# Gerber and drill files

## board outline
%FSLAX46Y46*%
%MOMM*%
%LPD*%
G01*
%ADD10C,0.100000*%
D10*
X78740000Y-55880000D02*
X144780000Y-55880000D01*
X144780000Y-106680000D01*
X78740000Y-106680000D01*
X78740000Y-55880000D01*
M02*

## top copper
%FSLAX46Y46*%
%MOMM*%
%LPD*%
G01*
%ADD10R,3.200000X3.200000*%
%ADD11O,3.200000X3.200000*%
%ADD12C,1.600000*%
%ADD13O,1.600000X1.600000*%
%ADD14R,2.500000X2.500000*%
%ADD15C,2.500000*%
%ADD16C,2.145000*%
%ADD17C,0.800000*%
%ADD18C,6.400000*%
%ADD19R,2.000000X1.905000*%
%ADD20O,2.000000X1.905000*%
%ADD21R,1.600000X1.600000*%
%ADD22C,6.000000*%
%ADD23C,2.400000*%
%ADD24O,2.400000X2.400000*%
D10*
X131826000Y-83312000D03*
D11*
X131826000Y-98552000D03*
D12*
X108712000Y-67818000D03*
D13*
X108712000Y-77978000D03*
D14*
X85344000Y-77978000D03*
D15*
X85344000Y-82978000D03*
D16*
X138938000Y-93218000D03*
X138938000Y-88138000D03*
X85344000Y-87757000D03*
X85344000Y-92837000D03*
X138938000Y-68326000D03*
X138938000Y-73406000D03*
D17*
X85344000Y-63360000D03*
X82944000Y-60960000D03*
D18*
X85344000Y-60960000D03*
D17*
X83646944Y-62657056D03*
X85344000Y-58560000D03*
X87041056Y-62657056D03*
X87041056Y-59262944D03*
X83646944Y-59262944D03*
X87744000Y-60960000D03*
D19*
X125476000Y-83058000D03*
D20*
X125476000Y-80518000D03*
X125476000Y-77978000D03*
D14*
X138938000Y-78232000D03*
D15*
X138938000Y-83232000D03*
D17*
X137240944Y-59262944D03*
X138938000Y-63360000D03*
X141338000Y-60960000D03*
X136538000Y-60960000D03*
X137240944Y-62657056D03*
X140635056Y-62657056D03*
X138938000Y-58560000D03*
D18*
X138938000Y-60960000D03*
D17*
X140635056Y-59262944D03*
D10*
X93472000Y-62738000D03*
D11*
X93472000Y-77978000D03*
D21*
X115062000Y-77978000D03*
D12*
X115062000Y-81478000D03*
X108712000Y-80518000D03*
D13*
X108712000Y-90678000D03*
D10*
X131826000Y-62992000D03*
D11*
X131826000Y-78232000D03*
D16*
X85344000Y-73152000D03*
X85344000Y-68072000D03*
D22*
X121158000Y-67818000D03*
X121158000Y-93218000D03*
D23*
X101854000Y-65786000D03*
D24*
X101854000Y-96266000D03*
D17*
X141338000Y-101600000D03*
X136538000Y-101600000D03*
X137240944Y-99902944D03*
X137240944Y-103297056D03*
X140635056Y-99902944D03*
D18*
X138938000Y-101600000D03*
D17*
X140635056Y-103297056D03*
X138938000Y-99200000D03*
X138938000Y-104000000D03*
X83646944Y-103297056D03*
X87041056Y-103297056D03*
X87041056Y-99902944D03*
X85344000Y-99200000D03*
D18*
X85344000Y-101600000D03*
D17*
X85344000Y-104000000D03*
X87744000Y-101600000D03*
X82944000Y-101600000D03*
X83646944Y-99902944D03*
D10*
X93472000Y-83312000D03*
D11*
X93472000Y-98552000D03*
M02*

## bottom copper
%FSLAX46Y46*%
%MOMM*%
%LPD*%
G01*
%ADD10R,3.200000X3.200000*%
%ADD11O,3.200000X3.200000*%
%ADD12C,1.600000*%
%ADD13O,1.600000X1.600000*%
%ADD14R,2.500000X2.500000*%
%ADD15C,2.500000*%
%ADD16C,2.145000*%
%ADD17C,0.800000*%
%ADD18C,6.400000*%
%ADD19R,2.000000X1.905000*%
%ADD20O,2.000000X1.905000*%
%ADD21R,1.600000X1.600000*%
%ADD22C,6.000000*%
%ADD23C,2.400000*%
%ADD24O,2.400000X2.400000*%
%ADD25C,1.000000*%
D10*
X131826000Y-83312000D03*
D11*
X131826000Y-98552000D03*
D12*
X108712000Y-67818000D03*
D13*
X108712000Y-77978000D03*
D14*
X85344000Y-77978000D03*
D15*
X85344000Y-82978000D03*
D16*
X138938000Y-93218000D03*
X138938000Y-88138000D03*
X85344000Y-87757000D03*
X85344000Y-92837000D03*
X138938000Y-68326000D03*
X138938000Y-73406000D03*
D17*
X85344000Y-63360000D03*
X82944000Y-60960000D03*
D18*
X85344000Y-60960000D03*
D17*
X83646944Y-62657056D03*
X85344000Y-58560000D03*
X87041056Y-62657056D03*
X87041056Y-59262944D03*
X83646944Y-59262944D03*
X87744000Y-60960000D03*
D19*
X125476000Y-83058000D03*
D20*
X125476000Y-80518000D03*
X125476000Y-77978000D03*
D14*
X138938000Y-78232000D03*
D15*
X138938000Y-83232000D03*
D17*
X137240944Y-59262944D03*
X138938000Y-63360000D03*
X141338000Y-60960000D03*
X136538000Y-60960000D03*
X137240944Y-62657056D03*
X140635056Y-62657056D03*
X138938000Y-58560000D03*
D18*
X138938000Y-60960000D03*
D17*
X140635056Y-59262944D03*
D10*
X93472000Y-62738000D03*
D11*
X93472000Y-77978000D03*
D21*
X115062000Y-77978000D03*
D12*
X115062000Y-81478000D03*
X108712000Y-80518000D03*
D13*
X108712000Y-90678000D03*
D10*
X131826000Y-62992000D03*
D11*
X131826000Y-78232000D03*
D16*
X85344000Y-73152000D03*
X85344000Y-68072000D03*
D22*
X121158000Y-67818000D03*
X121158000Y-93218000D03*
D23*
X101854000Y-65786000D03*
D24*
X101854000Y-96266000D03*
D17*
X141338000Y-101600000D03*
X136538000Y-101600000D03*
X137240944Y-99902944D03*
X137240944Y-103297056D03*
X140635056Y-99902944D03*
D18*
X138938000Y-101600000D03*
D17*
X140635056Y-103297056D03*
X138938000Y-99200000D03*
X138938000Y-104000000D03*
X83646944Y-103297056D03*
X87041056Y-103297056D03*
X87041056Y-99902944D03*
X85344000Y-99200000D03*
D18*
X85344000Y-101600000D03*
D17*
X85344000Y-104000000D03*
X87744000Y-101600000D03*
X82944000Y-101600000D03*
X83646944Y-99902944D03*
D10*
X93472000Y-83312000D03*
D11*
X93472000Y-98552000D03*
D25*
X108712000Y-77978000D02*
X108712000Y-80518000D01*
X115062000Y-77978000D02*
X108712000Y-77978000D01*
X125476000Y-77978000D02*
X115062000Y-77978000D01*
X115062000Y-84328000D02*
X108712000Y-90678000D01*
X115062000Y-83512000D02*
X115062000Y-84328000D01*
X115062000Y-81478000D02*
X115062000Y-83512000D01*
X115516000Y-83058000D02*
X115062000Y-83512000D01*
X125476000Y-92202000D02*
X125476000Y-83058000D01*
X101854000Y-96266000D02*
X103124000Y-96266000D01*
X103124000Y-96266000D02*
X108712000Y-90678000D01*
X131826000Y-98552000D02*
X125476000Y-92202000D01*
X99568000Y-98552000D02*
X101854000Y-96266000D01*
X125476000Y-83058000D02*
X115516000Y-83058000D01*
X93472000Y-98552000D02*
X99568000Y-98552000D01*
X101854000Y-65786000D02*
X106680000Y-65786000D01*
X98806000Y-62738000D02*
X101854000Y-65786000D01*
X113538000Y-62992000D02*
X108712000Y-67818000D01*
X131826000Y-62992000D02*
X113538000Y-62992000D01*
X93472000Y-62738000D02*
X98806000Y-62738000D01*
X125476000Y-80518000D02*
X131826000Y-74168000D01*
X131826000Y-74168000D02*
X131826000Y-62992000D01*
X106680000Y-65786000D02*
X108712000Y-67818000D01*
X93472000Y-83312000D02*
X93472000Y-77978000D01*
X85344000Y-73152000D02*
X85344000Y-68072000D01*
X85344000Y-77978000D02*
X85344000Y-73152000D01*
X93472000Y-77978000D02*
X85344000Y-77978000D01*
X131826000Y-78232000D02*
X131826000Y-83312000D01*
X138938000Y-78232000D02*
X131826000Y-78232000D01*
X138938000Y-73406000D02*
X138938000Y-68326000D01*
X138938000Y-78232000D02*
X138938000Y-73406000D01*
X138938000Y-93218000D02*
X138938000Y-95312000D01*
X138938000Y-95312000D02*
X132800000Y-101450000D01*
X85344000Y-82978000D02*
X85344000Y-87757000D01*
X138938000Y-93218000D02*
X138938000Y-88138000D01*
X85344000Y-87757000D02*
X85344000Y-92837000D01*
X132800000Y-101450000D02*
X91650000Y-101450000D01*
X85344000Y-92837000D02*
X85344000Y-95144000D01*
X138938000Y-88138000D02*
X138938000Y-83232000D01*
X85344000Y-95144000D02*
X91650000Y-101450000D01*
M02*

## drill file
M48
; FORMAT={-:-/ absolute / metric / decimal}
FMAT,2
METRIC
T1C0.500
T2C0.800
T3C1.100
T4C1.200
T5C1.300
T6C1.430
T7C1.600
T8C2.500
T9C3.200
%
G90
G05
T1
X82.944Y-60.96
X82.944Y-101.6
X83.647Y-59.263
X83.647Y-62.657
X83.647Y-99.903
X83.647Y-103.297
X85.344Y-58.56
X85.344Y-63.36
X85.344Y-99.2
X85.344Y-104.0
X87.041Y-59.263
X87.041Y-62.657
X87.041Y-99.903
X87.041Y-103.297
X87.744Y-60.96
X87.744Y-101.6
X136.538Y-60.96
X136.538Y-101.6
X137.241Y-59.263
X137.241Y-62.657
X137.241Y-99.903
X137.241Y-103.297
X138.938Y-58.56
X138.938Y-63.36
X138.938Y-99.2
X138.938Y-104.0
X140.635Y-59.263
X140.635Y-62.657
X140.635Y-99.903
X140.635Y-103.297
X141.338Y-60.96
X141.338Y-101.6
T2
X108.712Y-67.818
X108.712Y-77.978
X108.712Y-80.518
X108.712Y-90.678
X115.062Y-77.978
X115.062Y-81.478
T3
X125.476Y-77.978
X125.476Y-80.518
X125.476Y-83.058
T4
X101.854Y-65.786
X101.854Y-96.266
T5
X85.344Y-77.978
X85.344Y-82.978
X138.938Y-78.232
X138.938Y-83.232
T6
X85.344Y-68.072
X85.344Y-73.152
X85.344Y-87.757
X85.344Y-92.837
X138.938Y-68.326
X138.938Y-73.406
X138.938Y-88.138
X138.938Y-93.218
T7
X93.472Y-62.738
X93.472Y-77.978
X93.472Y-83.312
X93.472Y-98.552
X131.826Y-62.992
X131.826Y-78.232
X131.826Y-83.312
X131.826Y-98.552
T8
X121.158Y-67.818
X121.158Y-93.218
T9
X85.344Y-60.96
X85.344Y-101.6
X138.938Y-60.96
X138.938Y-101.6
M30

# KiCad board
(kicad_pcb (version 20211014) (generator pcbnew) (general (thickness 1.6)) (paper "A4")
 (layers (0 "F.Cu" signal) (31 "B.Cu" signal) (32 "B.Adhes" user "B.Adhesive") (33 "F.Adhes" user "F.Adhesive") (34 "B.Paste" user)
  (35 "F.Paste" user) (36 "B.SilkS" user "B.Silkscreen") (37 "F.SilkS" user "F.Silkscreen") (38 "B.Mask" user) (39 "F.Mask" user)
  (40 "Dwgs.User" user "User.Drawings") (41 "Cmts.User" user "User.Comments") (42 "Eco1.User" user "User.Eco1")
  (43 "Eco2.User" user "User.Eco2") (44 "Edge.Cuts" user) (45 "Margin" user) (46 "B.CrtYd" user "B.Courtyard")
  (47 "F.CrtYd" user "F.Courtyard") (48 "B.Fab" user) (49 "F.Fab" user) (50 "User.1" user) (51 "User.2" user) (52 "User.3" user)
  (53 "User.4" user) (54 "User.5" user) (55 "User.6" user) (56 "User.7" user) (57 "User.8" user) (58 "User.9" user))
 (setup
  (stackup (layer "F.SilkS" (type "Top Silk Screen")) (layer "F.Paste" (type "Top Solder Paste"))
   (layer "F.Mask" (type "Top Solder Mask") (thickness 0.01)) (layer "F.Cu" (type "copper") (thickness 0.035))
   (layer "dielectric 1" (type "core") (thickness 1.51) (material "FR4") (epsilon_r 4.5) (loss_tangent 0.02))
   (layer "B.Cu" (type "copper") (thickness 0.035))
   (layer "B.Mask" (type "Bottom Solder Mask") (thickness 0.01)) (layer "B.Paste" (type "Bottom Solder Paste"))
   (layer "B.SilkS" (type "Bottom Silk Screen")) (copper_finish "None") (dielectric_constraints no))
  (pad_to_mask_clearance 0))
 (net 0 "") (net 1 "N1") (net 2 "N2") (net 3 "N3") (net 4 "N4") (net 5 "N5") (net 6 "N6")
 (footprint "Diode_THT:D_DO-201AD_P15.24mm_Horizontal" (layer "F.Cu") (at 131.826 83.312 -90)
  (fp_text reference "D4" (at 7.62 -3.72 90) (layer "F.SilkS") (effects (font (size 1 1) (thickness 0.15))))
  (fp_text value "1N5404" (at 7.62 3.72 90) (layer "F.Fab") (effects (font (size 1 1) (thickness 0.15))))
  (pad "1" thru_hole rect (at 0 0 270) (size 3.2 3.2) (drill 1.6) (layers *.Cu *.Mask) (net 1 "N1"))
  (pad "2" thru_hole oval (at 15.24 0 270) (size 3.2 3.2) (drill 1.6) (layers *.Cu *.Mask) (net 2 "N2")))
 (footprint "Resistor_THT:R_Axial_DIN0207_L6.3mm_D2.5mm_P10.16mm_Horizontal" (layer "F.Cu") (at 108.712 67.818 -90)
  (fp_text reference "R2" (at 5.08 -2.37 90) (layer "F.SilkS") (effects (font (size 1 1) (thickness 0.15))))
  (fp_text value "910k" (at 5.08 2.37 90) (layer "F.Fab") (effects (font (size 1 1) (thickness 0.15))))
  (pad "1" thru_hole circle (at 0 0 270) (size 1.6 1.6) (drill 0.8) (layers *.Cu *.Mask) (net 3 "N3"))
  (pad "2" thru_hole oval (at 10.16 0 270) (size 1.6 1.6) (drill 0.8) (layers *.Cu *.Mask) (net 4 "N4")))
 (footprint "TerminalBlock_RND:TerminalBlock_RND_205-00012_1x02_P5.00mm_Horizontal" (layer "F.Cu") (at 85.344 77.978 -90)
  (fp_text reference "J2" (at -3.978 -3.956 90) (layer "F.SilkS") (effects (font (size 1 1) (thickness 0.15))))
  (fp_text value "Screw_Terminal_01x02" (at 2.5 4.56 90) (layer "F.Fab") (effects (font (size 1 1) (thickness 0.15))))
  (pad "1" thru_hole rect (at 0 0 270) (size 2.5 2.5) (drill 1.3) (layers *.Cu *.Mask) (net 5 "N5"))
  (pad "2" thru_hole circle (at 5 0 270) (size 2.5 2.5) (drill 1.3) (layers *.Cu *.Mask) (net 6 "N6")))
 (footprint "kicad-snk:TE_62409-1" (layer "F.Cu") (at 138.938 90.678 90)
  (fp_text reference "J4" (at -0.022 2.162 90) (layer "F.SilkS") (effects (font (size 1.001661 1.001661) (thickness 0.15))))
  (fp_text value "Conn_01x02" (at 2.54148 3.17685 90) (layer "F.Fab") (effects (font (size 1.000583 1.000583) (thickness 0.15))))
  (pad "1" thru_hole circle (at -2.54 0 90) (size 2.145 2.145) (drill 1.43) (layers *.Cu *.Mask) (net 6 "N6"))
  (pad "2" thru_hole circle (at 2.54 0 90) (size 2.145 2.145) (drill 1.43) (layers *.Cu *.Mask) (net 6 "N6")))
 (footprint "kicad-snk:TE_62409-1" (layer "F.Cu") (at 85.344 90.297 -90)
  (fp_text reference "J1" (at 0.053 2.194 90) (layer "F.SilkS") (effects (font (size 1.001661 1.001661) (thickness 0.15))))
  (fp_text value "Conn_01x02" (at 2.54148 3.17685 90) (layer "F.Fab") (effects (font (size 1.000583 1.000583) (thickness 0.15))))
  (pad "1" thru_hole circle (at -2.54 0 270) (size 2.145 2.145) (drill 1.43) (layers *.Cu *.Mask) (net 6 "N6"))
  (pad "2" thru_hole circle (at 2.54 0 270) (size 2.145 2.145) (drill 1.43) (layers *.Cu *.Mask) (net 6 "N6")))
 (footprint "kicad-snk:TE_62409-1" (layer "F.Cu") (at 138.938 70.866 -90)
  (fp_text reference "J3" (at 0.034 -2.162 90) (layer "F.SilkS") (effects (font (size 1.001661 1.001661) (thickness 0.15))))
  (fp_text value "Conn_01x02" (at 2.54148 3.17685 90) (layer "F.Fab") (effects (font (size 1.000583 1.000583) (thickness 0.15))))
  (pad "1" thru_hole circle (at -2.54 0 270) (size 2.145 2.145) (drill 1.43) (layers *.Cu *.Mask) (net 1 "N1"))
  (pad "2" thru_hole circle (at 2.54 0 270) (size 2.145 2.145) (drill 1.43) (layers *.Cu *.Mask) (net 1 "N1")))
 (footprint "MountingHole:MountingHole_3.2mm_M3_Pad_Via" (layer "F.Cu") (at 85.344 60.96)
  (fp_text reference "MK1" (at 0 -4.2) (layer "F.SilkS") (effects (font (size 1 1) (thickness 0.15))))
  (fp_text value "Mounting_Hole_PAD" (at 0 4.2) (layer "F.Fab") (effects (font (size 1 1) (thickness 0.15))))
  (pad "1" thru_hole circle (at 0 2.4) (size 0.8 0.8) (drill 0.5) (layers *.Cu *.Mask))
  (pad "1" thru_hole circle (at -2.4 0) (size 0.8 0.8) (drill 0.5) (layers *.Cu *.Mask))
  (pad "1" thru_hole circle (at 0 0) (size 6.4 6.4) (drill 3.2) (layers *.Cu *.Mask))
  (pad "1" thru_hole circle (at -1.697056 1.697056) (size 0.8 0.8) (drill 0.5) (layers *.Cu *.Mask))
  (pad "1" thru_hole circle (at 0 -2.4) (size 0.8 0.8) (drill 0.5) (layers *.Cu *.Mask))
  (pad "1" thru_hole circle (at 1.697056 1.697056) (size 0.8 0.8) (drill 0.5) (layers *.Cu *.Mask))
  (pad "1" thru_hole circle (at 1.697056 -1.697056) (size 0.8 0.8) (drill 0.5) (layers *.Cu *.Mask))
  (pad "1" thru_hole circle (at -1.697056 -1.697056) (size 0.8 0.8) (drill 0.5) (layers *.Cu *.Mask))
  (pad "1" thru_hole circle (at 2.4 0) (size 0.8 0.8) (drill 0.5) (layers *.Cu *.Mask)))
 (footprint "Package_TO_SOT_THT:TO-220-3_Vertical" (layer "F.Cu") (at 125.476 83.058 90)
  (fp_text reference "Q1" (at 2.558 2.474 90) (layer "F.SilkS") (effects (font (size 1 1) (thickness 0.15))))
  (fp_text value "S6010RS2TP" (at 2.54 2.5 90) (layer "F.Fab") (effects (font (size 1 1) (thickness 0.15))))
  (pad "1" thru_hole rect (at 0 0 90) (size 1.905 2) (drill 1.1) (layers *.Cu *.Mask) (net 2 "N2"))
  (pad "2" thru_hole oval (at 2.54 0 90) (size 1.905 2) (drill 1.1) (layers *.Cu *.Mask) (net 3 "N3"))
  (pad "3" thru_hole oval (at 5.08 0 90) (size 1.905 2) (drill 1.1) (layers *.Cu *.Mask) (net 4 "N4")))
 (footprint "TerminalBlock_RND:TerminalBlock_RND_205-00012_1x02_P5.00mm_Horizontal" (layer "F.Cu") (at 138.938 78.232 -90)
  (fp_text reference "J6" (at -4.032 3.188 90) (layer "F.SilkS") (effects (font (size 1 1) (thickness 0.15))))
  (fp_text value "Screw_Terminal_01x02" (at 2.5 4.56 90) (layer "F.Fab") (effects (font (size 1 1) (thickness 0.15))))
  (pad "1" thru_hole rect (at 0 0 270) (size 2.5 2.5) (drill 1.3) (layers *.Cu *.Mask) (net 1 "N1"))
  (pad "2" thru_hole circle (at 5 0 270) (size 2.5 2.5) (drill 1.3) (layers *.Cu *.Mask) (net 6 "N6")))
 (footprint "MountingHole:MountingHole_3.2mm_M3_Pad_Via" (layer "F.Cu") (at 138.938 60.96)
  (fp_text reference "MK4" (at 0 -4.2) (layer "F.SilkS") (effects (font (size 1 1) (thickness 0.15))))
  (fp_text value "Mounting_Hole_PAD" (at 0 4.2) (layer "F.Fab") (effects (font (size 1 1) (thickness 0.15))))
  (pad "1" thru_hole circle (at -1.697056 -1.697056) (size 0.8 0.8) (drill 0.5) (layers *.Cu *.Mask))
  (pad "1" thru_hole circle (at 0 2.4) (size 0.8 0.8) (drill 0.5) (layers *.Cu *.Mask))
  (pad "1" thru_hole circle (at 2.4 0) (size 0.8 0.8) (drill 0.5) (layers *.Cu *.Mask))
  (pad "1" thru_hole circle (at -2.4 0) (size 0.8 0.8) (drill 0.5) (layers *.Cu *.Mask))
  (pad "1" thru_hole circle (at -1.697056 1.697056) (size 0.8 0.8) (drill 0.5) (layers *.Cu *.Mask))
  (pad "1" thru_hole circle (at 1.697056 1.697056) (size 0.8 0.8) (drill 0.5) (layers *.Cu *.Mask))
  (pad "1" thru_hole circle (at 0 -2.4) (size 0.8 0.8) (drill 0.5) (layers *.Cu *.Mask))
  (pad "1" thru_hole circle (at 0 0) (size 6.4 6.4) (drill 3.2) (layers *.Cu *.Mask))
  (pad "1" thru_hole circle (at 1.697056 -1.697056) (size 0.8 0.8) (drill 0.5) (layers *.Cu *.Mask)))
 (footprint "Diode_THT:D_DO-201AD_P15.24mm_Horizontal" (layer "F.Cu") (at 93.472 62.738 -90)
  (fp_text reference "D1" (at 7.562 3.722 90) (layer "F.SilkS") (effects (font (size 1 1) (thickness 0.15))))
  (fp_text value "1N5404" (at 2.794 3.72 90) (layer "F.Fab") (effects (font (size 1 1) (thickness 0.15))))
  (pad "1" thru_hole rect (at 0 0 270) (size 3.2 3.2) (drill 1.6) (layers *.Cu *.Mask) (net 3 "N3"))
  (pad "2" thru_hole oval (at 15.24 0 270) (size 3.2 3.2) (drill 1.6) (layers *.Cu *.Mask) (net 5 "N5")))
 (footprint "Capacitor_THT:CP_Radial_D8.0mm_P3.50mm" (layer "F.Cu") (at 115.062 77.978 -90)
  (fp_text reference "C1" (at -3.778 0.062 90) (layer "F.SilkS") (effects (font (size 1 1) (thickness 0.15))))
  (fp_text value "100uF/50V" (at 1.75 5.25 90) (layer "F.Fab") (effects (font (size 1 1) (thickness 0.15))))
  (pad "1" thru_hole rect (at 0 0 270) (size 1.6 1.6) (drill 0.8) (layers *.Cu *.Mask) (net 4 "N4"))
  (pad "2" thru_hole circle (at 3.5 0 270) (size 1.6 1.6) (drill 0.8) (layers *.Cu *.Mask) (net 2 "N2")))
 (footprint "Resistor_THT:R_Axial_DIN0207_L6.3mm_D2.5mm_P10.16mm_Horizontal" (layer "F.Cu") (at 108.712 80.518 -90)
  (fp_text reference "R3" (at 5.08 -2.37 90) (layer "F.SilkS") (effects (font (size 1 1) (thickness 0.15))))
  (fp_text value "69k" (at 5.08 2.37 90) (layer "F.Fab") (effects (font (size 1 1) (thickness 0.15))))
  (pad "1" thru_hole circle (at 0 0 270) (size 1.6 1.6) (drill 0.8) (layers *.Cu *.Mask) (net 4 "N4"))
  (pad "2" thru_hole oval (at 10.16 0 270) (size 1.6 1.6) (drill 0.8) (layers *.Cu *.Mask) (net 2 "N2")))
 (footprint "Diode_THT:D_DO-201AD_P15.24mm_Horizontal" (layer "F.Cu") (at 131.826 62.992 -90)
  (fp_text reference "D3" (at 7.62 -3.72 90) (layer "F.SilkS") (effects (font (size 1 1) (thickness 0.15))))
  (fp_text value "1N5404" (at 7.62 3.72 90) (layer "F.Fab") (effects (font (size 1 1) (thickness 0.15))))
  (pad "1" thru_hole rect (at 0 0 270) (size 3.2 3.2) (drill 1.6) (layers *.Cu *.Mask) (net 3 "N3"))
  (pad "2" thru_hole oval (at 15.24 0 270) (size 3.2 3.2) (drill 1.6) (layers *.Cu *.Mask) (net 1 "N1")))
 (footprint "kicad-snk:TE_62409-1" (layer "F.Cu") (at 85.344 70.612 90)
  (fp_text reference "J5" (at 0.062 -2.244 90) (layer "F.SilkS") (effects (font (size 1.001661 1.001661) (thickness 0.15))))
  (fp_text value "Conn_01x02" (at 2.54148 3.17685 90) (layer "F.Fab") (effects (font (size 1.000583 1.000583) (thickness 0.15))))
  (pad "1" thru_hole circle (at -2.54 0 90) (size 2.145 2.145) (drill 1.43) (layers *.Cu *.Mask) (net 5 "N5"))
  (pad "2" thru_hole circle (at 2.54 0 90) (size 2.145 2.145) (drill 1.43) (layers *.Cu *.Mask) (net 5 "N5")))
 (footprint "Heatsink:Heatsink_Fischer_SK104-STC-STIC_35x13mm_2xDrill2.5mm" (layer "F.Cu") (at 121.158 80.518 90)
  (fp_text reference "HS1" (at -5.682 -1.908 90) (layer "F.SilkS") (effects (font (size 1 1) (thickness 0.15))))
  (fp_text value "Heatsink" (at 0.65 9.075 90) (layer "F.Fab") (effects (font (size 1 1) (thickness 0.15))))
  (pad "1" thru_hole circle (at 12.7 0 90) (size 6 6) (drill 2.5) (layers *.Cu *.Mask))
  (pad "1" thru_hole circle (at -12.7 0 270) (size 6 6) (drill 2.5) (layers *.Cu *.Mask)))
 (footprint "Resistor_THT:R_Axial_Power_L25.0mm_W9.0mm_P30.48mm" (layer "F.Cu") (at 101.854 65.786 -90)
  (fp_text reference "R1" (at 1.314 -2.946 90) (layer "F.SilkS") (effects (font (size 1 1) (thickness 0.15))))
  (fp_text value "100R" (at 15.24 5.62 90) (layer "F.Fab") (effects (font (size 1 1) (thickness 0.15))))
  (pad "1" thru_hole circle (at 0 0 270) (size 2.4 2.4) (drill 1.2) (layers *.Cu *.Mask) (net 3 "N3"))
  (pad "2" thru_hole oval (at 30.48 0 270) (size 2.4 2.4) (drill 1.2) (layers *.Cu *.Mask) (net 2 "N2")))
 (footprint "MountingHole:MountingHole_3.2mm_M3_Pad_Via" (layer "F.Cu") (at 138.938 101.6)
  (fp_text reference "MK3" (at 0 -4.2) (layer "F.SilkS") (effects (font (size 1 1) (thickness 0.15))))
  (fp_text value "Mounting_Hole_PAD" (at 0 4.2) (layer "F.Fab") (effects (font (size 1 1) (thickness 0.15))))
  (pad "1" thru_hole circle (at 2.4 0) (size 0.8 0.8) (drill 0.5) (layers *.Cu *.Mask))
  (pad "1" thru_hole circle (at -2.4 0) (size 0.8 0.8) (drill 0.5) (layers *.Cu *.Mask))
  (pad "1" thru_hole circle (at -1.697056 -1.697056) (size 0.8 0.8) (drill 0.5) (layers *.Cu *.Mask))
  (pad "1" thru_hole circle (at -1.697056 1.697056) (size 0.8 0.8) (drill 0.5) (layers *.Cu *.Mask))
  (pad "1" thru_hole circle (at 1.697056 -1.697056) (size 0.8 0.8) (drill 0.5) (layers *.Cu *.Mask))
  (pad "1" thru_hole circle (at 0 0) (size 6.4 6.4) (drill 3.2) (layers *.Cu *.Mask))
  (pad "1" thru_hole circle (at 1.697056 1.697056) (size 0.8 0.8) (drill 0.5) (layers *.Cu *.Mask))
  (pad "1" thru_hole circle (at 0 -2.4) (size 0.8 0.8) (drill 0.5) (layers *.Cu *.Mask))
  (pad "1" thru_hole circle (at 0 2.4) (size 0.8 0.8) (drill 0.5) (layers *.Cu *.Mask)))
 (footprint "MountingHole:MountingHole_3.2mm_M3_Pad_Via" (layer "F.Cu") (at 85.344 101.6)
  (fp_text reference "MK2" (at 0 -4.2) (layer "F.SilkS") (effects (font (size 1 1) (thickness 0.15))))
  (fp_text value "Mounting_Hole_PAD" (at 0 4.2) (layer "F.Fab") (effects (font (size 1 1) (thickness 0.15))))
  (pad "1" thru_hole circle (at -1.697056 1.697056) (size 0.8 0.8) (drill 0.5) (layers *.Cu *.Mask))
  (pad "1" thru_hole circle (at 1.697056 1.697056) (size 0.8 0.8) (drill 0.5) (layers *.Cu *.Mask))
  (pad "1" thru_hole circle (at 1.697056 -1.697056) (size 0.8 0.8) (drill 0.5) (layers *.Cu *.Mask))
  (pad "1" thru_hole circle (at 0 -2.4) (size 0.8 0.8) (drill 0.5) (layers *.Cu *.Mask))
  (pad "1" thru_hole circle (at 0 0) (size 6.4 6.4) (drill 3.2) (layers *.Cu *.Mask))
  (pad "1" thru_hole circle (at 0 2.4) (size 0.8 0.8) (drill 0.5) (layers *.Cu *.Mask))
  (pad "1" thru_hole circle (at 2.4 0) (size 0.8 0.8) (drill 0.5) (layers *.Cu *.Mask))
  (pad "1" thru_hole circle (at -2.4 0) (size 0.8 0.8) (drill 0.5) (layers *.Cu *.Mask))
  (pad "1" thru_hole circle (at -1.697056 -1.697056) (size 0.8 0.8) (drill 0.5) (layers *.Cu *.Mask)))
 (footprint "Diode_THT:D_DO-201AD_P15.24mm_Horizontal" (layer "F.Cu") (at 93.472 83.312 -90)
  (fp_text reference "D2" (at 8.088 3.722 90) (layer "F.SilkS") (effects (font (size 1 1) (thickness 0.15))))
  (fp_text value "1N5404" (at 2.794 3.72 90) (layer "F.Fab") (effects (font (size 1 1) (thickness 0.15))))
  (pad "1" thru_hole rect (at 0 0 270) (size 3.2 3.2) (drill 1.6) (layers *.Cu *.Mask) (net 5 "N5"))
  (pad "2" thru_hole oval (at 15.24 0 270) (size 3.2 3.2) (drill 1.6) (layers *.Cu *.Mask) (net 2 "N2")))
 (gr_rect (start 78.74 55.88) (end 144.78 106.68) (layer "Edge.Cuts") (width 0.1) (fill none))
 (segment (start 108.712 77.978) (end 108.712 80.518) (width 1) (layer "B.Cu") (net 4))
 (segment (start 115.062 77.978) (end 108.712 77.978) (width 1) (layer "B.Cu") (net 4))
 (segment (start 125.476 77.978) (end 115.062 77.978) (width 1) (layer "B.Cu") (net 4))
 (segment (start 115.062 84.328) (end 108.712 90.678) (width 1) (layer "B.Cu") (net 2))
 (segment (start 115.062 83.512) (end 115.062 84.328) (width 1) (layer "B.Cu") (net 2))
 (segment (start 115.062 81.478) (end 115.062 83.512) (width 1) (layer "B.Cu") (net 2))
 (segment (start 115.516 83.058) (end 115.062 83.512) (width 1) (layer "B.Cu") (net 2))
 (segment (start 125.476 92.202) (end 125.476 83.058) (width 1) (layer "B.Cu") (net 2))
 (segment (start 101.854 96.266) (end 103.124 96.266) (width 1) (layer "B.Cu") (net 2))
 (segment (start 103.124 96.266) (end 108.712 90.678) (width 1) (layer "B.Cu") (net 2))
 (segment (start 131.826 98.552) (end 125.476 92.202) (width 1) (layer "B.Cu") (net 2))
 (segment (start 99.568 98.552) (end 101.854 96.266) (width 1) (layer "B.Cu") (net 2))
 (segment (start 125.476 83.058) (end 115.516 83.058) (width 1) (layer "B.Cu") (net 2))
 (segment (start 93.472 98.552) (end 99.568 98.552) (width 1) (layer "B.Cu") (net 2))
 (segment (start 101.854 65.786) (end 106.68 65.786) (width 1) (layer "B.Cu") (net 3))
 (segment (start 98.806 62.738) (end 101.854 65.786) (width 1) (layer "B.Cu") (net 3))
 (segment (start 113.538 62.992) (end 108.712 67.818) (width 1) (layer "B.Cu") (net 3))
 (segment (start 131.826 62.992) (end 113.538 62.992) (width 1) (layer "B.Cu") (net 3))
 (segment (start 93.472 62.738) (end 98.806 62.738) (width 1) (layer "B.Cu") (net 3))
 (segment (start 125.476 80.518) (end 131.826 74.168) (width 1) (layer "B.Cu") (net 3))
 (segment (start 131.826 74.168) (end 131.826 62.992) (width 1) (layer "B.Cu") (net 3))
 (segment (start 106.68 65.786) (end 108.712 67.818) (width 1) (layer "B.Cu") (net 3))
 (segment (start 93.472 83.312) (end 93.472 77.978) (width 1) (layer "B.Cu") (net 5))
 (segment (start 85.344 73.152) (end 85.344 68.072) (width 1) (layer "B.Cu") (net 5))
 (segment (start 85.344 77.978) (end 85.344 73.152) (width 1) (layer "B.Cu") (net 5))
 (segment (start 93.472 77.978) (end 85.344 77.978) (width 1) (layer "B.Cu") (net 5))
 (segment (start 131.826 78.232) (end 131.826 83.312) (width 1) (layer "B.Cu") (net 1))
 (segment (start 138.938 78.232) (end 131.826 78.232) (width 1) (layer "B.Cu") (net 1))
 (segment (start 138.938 73.406) (end 138.938 68.326) (width 1) (layer "B.Cu") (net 1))
 (segment (start 138.938 78.232) (end 138.938 73.406) (width 1) (layer "B.Cu") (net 1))
 (segment (start 138.938 93.218) (end 138.938 95.312) (width 1) (layer "B.Cu") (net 6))
 (segment (start 138.938 95.312) (end 132.8 101.45) (width 1) (layer "B.Cu") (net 6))
 (segment (start 85.344 82.978) (end 85.344 87.757) (width 1) (layer "B.Cu") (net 6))
 (segment (start 138.938 93.218) (end 138.938 88.138) (width 1) (layer "B.Cu") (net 6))
 (segment (start 85.344 87.757) (end 85.344 92.837) (width 1) (layer "B.Cu") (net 6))
 (segment (start 132.8 101.45) (end 91.65 101.45) (width 1) (layer "B.Cu") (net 6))
 (segment (start 85.344 92.837) (end 85.344 95.144) (width 1) (layer "B.Cu") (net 6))
 (segment (start 138.938 88.138) (end 138.938 83.232) (width 1) (layer "B.Cu") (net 6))
 (segment (start 85.344 95.144) (end 91.65 101.45) (width 1) (layer "B.Cu") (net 6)))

